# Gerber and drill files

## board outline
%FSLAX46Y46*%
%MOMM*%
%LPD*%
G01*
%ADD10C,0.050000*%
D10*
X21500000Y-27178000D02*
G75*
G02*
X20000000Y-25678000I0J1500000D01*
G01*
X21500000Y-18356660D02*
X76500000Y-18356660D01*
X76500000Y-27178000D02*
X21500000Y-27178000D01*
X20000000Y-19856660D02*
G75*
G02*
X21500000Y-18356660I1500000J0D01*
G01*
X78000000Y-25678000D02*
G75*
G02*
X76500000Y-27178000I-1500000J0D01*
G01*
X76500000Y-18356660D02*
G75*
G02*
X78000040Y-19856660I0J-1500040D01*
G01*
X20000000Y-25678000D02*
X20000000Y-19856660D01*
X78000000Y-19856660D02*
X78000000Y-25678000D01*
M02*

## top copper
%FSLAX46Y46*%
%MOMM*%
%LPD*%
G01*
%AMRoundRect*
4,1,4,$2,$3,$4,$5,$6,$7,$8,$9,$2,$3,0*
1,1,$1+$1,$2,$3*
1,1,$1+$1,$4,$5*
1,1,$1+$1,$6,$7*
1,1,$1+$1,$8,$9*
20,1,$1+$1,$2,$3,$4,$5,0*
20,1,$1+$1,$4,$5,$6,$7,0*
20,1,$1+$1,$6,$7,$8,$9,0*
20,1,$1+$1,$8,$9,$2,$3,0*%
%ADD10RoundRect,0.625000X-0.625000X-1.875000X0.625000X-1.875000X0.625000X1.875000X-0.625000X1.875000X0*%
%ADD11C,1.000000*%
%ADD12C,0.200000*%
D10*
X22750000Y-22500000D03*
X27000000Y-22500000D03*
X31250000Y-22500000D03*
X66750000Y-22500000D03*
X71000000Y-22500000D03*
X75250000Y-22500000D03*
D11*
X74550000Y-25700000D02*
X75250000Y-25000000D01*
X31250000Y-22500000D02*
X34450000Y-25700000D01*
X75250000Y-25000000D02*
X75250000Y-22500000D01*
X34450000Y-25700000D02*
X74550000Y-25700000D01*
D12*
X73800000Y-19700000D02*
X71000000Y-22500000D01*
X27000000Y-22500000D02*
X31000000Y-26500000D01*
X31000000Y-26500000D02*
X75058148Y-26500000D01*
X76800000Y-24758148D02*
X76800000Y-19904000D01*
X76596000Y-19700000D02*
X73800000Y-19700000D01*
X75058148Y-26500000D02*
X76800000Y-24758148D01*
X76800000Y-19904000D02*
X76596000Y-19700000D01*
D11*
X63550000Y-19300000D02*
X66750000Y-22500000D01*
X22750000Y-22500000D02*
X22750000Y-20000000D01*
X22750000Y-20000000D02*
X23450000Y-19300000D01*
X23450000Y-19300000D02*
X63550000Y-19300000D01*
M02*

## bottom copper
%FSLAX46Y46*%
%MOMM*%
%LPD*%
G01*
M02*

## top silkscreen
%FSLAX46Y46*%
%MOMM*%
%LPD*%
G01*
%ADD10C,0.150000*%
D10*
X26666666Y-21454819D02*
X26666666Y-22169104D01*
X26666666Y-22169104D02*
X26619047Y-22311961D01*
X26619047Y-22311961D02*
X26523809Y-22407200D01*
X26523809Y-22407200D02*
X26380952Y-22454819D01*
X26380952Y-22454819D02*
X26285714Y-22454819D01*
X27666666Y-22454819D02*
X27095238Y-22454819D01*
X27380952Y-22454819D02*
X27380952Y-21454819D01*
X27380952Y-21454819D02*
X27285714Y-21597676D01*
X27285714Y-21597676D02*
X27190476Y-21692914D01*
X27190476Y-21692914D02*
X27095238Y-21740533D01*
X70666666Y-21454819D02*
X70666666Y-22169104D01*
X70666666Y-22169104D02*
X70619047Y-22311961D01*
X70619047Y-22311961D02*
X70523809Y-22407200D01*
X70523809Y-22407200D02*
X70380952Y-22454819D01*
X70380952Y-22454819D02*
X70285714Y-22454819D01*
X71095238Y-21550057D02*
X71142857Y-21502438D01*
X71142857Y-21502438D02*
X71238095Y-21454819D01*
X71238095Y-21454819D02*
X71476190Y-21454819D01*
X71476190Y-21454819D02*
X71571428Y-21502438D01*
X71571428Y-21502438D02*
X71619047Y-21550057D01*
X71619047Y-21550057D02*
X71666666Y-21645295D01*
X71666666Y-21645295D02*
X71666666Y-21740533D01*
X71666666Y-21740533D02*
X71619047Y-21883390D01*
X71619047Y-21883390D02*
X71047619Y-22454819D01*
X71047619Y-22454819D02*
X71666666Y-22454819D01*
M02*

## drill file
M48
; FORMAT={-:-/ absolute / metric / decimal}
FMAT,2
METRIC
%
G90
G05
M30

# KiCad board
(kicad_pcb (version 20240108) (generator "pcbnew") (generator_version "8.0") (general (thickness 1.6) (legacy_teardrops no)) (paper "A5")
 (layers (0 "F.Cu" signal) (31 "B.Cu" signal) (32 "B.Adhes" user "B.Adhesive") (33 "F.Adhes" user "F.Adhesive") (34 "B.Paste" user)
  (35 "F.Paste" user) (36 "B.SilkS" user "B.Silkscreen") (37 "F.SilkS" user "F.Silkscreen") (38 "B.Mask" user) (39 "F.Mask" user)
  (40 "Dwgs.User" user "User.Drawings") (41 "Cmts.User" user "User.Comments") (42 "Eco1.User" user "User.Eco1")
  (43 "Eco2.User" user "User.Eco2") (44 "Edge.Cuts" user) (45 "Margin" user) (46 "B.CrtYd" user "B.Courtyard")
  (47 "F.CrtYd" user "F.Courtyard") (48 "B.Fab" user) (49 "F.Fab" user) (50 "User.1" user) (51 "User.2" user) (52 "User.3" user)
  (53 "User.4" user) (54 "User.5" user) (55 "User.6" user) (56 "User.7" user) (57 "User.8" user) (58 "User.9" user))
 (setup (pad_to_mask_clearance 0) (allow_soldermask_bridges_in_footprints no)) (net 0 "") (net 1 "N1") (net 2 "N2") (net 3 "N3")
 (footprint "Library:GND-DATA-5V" (layer "F.Cu") (at 27 22.5)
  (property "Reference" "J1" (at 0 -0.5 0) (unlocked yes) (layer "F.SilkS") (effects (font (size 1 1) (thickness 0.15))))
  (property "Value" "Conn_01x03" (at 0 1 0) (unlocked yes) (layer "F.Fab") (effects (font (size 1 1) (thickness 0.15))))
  (pad "1" smd roundrect (at -4.25 0) (size 2.5 5) (layers "F.Cu" "F.Paste" "F.Mask") (roundrect_rratio 0.25) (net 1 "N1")
   (thermal_bridge_angle 45))
  (pad "2" smd roundrect (at 0 0) (size 2.5 5) (layers "F.Cu" "F.Paste" "F.Mask") (roundrect_rratio 0.25) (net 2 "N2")
   (thermal_bridge_angle 45))
  (pad "3" smd roundrect (at 4.25 0) (size 2.5 5) (layers "F.Cu" "F.Paste" "F.Mask") (roundrect_rratio 0.25) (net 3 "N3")
   (thermal_bridge_angle 45)))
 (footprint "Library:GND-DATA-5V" (layer "F.Cu") (at 71 22.5)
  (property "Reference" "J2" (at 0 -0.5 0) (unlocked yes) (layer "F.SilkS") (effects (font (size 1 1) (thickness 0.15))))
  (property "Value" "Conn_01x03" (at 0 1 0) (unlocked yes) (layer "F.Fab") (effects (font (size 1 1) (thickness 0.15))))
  (pad "1" smd roundrect (at -4.25 0) (size 2.5 5) (layers "F.Cu" "F.Paste" "F.Mask") (roundrect_rratio 0.25) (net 1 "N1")
   (thermal_bridge_angle 45))
  (pad "2" smd roundrect (at 0 0) (size 2.5 5) (layers "F.Cu" "F.Paste" "F.Mask") (roundrect_rratio 0.25) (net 2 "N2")
   (thermal_bridge_angle 45))
  (pad "3" smd roundrect (at 4.25 0) (size 2.5 5) (layers "F.Cu" "F.Paste" "F.Mask") (roundrect_rratio 0.25) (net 3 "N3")
   (thermal_bridge_angle 45)))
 (gr_arc (start 21.5 27.178) (mid 20.43934 26.73866) (end 20 25.678) (stroke (width 0.05) (type default)) (layer "Edge.Cuts"))
 (gr_line (start 21.5 18.35666) (end 76.5 18.35666) (stroke (width 0.05) (type default)) (layer "Edge.Cuts"))
 (gr_line (start 76.5 27.178) (end 21.5 27.178) (stroke (width 0.05) (type default)) (layer "Edge.Cuts"))
 (gr_arc (start 20 19.85666) (mid 20.43934 18.796) (end 21.5 18.35666) (stroke (width 0.05) (type default)) (layer "Edge.Cuts"))
 (gr_arc (start 78 25.678) (mid 77.56066 26.73866) (end 76.5 27.178) (stroke (width 0.05) (type default)) (layer "Edge.Cuts"))
 (gr_arc (start 76.5 18.35666) (mid 77.56066 18.796) (end 78 19.85666) (stroke (width 0.05) (type default)) (layer "Edge.Cuts"))
 (gr_line (start 20 25.678) (end 20 19.85666) (stroke (width 0.05) (type default)) (layer "Edge.Cuts"))
 (gr_line (start 78 19.85666) (end 78 25.678) (stroke (width 0.05) (type default)) (layer "Edge.Cuts"))
 (segment (start 74.55 25.7) (end 75.25 25) (width 1) (layer "F.Cu") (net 3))
 (segment (start 31.25 22.5) (end 34.45 25.7) (width 1) (layer "F.Cu") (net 3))
 (segment (start 75.25 25) (end 75.25 22.5) (width 1) (layer "F.Cu") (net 3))
 (segment (start 34.45 25.7) (end 74.55 25.7) (width 1) (layer "F.Cu") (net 3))
 (segment (start 73.8 19.7) (end 71 22.5) (width 0.2) (layer "F.Cu") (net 2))
 (segment (start 27 22.5) (end 31 26.5) (width 0.2) (layer "F.Cu") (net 2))
 (segment (start 31 26.5) (end 75.058148 26.5) (width 0.2) (layer "F.Cu") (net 2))
 (segment (start 76.8 24.758148) (end 76.8 19.904) (width 0.2) (layer "F.Cu") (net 2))
 (segment (start 76.596 19.7) (end 73.8 19.7) (width 0.2) (layer "F.Cu") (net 2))
 (segment (start 75.058148 26.5) (end 76.8 24.758148) (width 0.2) (layer "F.Cu") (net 2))
 (segment (start 76.8 19.904) (end 76.596 19.7) (width 0.2) (layer "F.Cu") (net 2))
 (segment (start 63.55 19.3) (end 66.75 22.5) (width 1) (layer "F.Cu") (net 1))
 (segment (start 22.75 22.5) (end 22.75 20) (width 1) (layer "F.Cu") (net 1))
 (segment (start 22.75 20) (end 23.45 19.3) (width 1) (layer "F.Cu") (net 1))
 (segment (start 23.45 19.3) (end 63.55 19.3) (width 1) (layer "F.Cu") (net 1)))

